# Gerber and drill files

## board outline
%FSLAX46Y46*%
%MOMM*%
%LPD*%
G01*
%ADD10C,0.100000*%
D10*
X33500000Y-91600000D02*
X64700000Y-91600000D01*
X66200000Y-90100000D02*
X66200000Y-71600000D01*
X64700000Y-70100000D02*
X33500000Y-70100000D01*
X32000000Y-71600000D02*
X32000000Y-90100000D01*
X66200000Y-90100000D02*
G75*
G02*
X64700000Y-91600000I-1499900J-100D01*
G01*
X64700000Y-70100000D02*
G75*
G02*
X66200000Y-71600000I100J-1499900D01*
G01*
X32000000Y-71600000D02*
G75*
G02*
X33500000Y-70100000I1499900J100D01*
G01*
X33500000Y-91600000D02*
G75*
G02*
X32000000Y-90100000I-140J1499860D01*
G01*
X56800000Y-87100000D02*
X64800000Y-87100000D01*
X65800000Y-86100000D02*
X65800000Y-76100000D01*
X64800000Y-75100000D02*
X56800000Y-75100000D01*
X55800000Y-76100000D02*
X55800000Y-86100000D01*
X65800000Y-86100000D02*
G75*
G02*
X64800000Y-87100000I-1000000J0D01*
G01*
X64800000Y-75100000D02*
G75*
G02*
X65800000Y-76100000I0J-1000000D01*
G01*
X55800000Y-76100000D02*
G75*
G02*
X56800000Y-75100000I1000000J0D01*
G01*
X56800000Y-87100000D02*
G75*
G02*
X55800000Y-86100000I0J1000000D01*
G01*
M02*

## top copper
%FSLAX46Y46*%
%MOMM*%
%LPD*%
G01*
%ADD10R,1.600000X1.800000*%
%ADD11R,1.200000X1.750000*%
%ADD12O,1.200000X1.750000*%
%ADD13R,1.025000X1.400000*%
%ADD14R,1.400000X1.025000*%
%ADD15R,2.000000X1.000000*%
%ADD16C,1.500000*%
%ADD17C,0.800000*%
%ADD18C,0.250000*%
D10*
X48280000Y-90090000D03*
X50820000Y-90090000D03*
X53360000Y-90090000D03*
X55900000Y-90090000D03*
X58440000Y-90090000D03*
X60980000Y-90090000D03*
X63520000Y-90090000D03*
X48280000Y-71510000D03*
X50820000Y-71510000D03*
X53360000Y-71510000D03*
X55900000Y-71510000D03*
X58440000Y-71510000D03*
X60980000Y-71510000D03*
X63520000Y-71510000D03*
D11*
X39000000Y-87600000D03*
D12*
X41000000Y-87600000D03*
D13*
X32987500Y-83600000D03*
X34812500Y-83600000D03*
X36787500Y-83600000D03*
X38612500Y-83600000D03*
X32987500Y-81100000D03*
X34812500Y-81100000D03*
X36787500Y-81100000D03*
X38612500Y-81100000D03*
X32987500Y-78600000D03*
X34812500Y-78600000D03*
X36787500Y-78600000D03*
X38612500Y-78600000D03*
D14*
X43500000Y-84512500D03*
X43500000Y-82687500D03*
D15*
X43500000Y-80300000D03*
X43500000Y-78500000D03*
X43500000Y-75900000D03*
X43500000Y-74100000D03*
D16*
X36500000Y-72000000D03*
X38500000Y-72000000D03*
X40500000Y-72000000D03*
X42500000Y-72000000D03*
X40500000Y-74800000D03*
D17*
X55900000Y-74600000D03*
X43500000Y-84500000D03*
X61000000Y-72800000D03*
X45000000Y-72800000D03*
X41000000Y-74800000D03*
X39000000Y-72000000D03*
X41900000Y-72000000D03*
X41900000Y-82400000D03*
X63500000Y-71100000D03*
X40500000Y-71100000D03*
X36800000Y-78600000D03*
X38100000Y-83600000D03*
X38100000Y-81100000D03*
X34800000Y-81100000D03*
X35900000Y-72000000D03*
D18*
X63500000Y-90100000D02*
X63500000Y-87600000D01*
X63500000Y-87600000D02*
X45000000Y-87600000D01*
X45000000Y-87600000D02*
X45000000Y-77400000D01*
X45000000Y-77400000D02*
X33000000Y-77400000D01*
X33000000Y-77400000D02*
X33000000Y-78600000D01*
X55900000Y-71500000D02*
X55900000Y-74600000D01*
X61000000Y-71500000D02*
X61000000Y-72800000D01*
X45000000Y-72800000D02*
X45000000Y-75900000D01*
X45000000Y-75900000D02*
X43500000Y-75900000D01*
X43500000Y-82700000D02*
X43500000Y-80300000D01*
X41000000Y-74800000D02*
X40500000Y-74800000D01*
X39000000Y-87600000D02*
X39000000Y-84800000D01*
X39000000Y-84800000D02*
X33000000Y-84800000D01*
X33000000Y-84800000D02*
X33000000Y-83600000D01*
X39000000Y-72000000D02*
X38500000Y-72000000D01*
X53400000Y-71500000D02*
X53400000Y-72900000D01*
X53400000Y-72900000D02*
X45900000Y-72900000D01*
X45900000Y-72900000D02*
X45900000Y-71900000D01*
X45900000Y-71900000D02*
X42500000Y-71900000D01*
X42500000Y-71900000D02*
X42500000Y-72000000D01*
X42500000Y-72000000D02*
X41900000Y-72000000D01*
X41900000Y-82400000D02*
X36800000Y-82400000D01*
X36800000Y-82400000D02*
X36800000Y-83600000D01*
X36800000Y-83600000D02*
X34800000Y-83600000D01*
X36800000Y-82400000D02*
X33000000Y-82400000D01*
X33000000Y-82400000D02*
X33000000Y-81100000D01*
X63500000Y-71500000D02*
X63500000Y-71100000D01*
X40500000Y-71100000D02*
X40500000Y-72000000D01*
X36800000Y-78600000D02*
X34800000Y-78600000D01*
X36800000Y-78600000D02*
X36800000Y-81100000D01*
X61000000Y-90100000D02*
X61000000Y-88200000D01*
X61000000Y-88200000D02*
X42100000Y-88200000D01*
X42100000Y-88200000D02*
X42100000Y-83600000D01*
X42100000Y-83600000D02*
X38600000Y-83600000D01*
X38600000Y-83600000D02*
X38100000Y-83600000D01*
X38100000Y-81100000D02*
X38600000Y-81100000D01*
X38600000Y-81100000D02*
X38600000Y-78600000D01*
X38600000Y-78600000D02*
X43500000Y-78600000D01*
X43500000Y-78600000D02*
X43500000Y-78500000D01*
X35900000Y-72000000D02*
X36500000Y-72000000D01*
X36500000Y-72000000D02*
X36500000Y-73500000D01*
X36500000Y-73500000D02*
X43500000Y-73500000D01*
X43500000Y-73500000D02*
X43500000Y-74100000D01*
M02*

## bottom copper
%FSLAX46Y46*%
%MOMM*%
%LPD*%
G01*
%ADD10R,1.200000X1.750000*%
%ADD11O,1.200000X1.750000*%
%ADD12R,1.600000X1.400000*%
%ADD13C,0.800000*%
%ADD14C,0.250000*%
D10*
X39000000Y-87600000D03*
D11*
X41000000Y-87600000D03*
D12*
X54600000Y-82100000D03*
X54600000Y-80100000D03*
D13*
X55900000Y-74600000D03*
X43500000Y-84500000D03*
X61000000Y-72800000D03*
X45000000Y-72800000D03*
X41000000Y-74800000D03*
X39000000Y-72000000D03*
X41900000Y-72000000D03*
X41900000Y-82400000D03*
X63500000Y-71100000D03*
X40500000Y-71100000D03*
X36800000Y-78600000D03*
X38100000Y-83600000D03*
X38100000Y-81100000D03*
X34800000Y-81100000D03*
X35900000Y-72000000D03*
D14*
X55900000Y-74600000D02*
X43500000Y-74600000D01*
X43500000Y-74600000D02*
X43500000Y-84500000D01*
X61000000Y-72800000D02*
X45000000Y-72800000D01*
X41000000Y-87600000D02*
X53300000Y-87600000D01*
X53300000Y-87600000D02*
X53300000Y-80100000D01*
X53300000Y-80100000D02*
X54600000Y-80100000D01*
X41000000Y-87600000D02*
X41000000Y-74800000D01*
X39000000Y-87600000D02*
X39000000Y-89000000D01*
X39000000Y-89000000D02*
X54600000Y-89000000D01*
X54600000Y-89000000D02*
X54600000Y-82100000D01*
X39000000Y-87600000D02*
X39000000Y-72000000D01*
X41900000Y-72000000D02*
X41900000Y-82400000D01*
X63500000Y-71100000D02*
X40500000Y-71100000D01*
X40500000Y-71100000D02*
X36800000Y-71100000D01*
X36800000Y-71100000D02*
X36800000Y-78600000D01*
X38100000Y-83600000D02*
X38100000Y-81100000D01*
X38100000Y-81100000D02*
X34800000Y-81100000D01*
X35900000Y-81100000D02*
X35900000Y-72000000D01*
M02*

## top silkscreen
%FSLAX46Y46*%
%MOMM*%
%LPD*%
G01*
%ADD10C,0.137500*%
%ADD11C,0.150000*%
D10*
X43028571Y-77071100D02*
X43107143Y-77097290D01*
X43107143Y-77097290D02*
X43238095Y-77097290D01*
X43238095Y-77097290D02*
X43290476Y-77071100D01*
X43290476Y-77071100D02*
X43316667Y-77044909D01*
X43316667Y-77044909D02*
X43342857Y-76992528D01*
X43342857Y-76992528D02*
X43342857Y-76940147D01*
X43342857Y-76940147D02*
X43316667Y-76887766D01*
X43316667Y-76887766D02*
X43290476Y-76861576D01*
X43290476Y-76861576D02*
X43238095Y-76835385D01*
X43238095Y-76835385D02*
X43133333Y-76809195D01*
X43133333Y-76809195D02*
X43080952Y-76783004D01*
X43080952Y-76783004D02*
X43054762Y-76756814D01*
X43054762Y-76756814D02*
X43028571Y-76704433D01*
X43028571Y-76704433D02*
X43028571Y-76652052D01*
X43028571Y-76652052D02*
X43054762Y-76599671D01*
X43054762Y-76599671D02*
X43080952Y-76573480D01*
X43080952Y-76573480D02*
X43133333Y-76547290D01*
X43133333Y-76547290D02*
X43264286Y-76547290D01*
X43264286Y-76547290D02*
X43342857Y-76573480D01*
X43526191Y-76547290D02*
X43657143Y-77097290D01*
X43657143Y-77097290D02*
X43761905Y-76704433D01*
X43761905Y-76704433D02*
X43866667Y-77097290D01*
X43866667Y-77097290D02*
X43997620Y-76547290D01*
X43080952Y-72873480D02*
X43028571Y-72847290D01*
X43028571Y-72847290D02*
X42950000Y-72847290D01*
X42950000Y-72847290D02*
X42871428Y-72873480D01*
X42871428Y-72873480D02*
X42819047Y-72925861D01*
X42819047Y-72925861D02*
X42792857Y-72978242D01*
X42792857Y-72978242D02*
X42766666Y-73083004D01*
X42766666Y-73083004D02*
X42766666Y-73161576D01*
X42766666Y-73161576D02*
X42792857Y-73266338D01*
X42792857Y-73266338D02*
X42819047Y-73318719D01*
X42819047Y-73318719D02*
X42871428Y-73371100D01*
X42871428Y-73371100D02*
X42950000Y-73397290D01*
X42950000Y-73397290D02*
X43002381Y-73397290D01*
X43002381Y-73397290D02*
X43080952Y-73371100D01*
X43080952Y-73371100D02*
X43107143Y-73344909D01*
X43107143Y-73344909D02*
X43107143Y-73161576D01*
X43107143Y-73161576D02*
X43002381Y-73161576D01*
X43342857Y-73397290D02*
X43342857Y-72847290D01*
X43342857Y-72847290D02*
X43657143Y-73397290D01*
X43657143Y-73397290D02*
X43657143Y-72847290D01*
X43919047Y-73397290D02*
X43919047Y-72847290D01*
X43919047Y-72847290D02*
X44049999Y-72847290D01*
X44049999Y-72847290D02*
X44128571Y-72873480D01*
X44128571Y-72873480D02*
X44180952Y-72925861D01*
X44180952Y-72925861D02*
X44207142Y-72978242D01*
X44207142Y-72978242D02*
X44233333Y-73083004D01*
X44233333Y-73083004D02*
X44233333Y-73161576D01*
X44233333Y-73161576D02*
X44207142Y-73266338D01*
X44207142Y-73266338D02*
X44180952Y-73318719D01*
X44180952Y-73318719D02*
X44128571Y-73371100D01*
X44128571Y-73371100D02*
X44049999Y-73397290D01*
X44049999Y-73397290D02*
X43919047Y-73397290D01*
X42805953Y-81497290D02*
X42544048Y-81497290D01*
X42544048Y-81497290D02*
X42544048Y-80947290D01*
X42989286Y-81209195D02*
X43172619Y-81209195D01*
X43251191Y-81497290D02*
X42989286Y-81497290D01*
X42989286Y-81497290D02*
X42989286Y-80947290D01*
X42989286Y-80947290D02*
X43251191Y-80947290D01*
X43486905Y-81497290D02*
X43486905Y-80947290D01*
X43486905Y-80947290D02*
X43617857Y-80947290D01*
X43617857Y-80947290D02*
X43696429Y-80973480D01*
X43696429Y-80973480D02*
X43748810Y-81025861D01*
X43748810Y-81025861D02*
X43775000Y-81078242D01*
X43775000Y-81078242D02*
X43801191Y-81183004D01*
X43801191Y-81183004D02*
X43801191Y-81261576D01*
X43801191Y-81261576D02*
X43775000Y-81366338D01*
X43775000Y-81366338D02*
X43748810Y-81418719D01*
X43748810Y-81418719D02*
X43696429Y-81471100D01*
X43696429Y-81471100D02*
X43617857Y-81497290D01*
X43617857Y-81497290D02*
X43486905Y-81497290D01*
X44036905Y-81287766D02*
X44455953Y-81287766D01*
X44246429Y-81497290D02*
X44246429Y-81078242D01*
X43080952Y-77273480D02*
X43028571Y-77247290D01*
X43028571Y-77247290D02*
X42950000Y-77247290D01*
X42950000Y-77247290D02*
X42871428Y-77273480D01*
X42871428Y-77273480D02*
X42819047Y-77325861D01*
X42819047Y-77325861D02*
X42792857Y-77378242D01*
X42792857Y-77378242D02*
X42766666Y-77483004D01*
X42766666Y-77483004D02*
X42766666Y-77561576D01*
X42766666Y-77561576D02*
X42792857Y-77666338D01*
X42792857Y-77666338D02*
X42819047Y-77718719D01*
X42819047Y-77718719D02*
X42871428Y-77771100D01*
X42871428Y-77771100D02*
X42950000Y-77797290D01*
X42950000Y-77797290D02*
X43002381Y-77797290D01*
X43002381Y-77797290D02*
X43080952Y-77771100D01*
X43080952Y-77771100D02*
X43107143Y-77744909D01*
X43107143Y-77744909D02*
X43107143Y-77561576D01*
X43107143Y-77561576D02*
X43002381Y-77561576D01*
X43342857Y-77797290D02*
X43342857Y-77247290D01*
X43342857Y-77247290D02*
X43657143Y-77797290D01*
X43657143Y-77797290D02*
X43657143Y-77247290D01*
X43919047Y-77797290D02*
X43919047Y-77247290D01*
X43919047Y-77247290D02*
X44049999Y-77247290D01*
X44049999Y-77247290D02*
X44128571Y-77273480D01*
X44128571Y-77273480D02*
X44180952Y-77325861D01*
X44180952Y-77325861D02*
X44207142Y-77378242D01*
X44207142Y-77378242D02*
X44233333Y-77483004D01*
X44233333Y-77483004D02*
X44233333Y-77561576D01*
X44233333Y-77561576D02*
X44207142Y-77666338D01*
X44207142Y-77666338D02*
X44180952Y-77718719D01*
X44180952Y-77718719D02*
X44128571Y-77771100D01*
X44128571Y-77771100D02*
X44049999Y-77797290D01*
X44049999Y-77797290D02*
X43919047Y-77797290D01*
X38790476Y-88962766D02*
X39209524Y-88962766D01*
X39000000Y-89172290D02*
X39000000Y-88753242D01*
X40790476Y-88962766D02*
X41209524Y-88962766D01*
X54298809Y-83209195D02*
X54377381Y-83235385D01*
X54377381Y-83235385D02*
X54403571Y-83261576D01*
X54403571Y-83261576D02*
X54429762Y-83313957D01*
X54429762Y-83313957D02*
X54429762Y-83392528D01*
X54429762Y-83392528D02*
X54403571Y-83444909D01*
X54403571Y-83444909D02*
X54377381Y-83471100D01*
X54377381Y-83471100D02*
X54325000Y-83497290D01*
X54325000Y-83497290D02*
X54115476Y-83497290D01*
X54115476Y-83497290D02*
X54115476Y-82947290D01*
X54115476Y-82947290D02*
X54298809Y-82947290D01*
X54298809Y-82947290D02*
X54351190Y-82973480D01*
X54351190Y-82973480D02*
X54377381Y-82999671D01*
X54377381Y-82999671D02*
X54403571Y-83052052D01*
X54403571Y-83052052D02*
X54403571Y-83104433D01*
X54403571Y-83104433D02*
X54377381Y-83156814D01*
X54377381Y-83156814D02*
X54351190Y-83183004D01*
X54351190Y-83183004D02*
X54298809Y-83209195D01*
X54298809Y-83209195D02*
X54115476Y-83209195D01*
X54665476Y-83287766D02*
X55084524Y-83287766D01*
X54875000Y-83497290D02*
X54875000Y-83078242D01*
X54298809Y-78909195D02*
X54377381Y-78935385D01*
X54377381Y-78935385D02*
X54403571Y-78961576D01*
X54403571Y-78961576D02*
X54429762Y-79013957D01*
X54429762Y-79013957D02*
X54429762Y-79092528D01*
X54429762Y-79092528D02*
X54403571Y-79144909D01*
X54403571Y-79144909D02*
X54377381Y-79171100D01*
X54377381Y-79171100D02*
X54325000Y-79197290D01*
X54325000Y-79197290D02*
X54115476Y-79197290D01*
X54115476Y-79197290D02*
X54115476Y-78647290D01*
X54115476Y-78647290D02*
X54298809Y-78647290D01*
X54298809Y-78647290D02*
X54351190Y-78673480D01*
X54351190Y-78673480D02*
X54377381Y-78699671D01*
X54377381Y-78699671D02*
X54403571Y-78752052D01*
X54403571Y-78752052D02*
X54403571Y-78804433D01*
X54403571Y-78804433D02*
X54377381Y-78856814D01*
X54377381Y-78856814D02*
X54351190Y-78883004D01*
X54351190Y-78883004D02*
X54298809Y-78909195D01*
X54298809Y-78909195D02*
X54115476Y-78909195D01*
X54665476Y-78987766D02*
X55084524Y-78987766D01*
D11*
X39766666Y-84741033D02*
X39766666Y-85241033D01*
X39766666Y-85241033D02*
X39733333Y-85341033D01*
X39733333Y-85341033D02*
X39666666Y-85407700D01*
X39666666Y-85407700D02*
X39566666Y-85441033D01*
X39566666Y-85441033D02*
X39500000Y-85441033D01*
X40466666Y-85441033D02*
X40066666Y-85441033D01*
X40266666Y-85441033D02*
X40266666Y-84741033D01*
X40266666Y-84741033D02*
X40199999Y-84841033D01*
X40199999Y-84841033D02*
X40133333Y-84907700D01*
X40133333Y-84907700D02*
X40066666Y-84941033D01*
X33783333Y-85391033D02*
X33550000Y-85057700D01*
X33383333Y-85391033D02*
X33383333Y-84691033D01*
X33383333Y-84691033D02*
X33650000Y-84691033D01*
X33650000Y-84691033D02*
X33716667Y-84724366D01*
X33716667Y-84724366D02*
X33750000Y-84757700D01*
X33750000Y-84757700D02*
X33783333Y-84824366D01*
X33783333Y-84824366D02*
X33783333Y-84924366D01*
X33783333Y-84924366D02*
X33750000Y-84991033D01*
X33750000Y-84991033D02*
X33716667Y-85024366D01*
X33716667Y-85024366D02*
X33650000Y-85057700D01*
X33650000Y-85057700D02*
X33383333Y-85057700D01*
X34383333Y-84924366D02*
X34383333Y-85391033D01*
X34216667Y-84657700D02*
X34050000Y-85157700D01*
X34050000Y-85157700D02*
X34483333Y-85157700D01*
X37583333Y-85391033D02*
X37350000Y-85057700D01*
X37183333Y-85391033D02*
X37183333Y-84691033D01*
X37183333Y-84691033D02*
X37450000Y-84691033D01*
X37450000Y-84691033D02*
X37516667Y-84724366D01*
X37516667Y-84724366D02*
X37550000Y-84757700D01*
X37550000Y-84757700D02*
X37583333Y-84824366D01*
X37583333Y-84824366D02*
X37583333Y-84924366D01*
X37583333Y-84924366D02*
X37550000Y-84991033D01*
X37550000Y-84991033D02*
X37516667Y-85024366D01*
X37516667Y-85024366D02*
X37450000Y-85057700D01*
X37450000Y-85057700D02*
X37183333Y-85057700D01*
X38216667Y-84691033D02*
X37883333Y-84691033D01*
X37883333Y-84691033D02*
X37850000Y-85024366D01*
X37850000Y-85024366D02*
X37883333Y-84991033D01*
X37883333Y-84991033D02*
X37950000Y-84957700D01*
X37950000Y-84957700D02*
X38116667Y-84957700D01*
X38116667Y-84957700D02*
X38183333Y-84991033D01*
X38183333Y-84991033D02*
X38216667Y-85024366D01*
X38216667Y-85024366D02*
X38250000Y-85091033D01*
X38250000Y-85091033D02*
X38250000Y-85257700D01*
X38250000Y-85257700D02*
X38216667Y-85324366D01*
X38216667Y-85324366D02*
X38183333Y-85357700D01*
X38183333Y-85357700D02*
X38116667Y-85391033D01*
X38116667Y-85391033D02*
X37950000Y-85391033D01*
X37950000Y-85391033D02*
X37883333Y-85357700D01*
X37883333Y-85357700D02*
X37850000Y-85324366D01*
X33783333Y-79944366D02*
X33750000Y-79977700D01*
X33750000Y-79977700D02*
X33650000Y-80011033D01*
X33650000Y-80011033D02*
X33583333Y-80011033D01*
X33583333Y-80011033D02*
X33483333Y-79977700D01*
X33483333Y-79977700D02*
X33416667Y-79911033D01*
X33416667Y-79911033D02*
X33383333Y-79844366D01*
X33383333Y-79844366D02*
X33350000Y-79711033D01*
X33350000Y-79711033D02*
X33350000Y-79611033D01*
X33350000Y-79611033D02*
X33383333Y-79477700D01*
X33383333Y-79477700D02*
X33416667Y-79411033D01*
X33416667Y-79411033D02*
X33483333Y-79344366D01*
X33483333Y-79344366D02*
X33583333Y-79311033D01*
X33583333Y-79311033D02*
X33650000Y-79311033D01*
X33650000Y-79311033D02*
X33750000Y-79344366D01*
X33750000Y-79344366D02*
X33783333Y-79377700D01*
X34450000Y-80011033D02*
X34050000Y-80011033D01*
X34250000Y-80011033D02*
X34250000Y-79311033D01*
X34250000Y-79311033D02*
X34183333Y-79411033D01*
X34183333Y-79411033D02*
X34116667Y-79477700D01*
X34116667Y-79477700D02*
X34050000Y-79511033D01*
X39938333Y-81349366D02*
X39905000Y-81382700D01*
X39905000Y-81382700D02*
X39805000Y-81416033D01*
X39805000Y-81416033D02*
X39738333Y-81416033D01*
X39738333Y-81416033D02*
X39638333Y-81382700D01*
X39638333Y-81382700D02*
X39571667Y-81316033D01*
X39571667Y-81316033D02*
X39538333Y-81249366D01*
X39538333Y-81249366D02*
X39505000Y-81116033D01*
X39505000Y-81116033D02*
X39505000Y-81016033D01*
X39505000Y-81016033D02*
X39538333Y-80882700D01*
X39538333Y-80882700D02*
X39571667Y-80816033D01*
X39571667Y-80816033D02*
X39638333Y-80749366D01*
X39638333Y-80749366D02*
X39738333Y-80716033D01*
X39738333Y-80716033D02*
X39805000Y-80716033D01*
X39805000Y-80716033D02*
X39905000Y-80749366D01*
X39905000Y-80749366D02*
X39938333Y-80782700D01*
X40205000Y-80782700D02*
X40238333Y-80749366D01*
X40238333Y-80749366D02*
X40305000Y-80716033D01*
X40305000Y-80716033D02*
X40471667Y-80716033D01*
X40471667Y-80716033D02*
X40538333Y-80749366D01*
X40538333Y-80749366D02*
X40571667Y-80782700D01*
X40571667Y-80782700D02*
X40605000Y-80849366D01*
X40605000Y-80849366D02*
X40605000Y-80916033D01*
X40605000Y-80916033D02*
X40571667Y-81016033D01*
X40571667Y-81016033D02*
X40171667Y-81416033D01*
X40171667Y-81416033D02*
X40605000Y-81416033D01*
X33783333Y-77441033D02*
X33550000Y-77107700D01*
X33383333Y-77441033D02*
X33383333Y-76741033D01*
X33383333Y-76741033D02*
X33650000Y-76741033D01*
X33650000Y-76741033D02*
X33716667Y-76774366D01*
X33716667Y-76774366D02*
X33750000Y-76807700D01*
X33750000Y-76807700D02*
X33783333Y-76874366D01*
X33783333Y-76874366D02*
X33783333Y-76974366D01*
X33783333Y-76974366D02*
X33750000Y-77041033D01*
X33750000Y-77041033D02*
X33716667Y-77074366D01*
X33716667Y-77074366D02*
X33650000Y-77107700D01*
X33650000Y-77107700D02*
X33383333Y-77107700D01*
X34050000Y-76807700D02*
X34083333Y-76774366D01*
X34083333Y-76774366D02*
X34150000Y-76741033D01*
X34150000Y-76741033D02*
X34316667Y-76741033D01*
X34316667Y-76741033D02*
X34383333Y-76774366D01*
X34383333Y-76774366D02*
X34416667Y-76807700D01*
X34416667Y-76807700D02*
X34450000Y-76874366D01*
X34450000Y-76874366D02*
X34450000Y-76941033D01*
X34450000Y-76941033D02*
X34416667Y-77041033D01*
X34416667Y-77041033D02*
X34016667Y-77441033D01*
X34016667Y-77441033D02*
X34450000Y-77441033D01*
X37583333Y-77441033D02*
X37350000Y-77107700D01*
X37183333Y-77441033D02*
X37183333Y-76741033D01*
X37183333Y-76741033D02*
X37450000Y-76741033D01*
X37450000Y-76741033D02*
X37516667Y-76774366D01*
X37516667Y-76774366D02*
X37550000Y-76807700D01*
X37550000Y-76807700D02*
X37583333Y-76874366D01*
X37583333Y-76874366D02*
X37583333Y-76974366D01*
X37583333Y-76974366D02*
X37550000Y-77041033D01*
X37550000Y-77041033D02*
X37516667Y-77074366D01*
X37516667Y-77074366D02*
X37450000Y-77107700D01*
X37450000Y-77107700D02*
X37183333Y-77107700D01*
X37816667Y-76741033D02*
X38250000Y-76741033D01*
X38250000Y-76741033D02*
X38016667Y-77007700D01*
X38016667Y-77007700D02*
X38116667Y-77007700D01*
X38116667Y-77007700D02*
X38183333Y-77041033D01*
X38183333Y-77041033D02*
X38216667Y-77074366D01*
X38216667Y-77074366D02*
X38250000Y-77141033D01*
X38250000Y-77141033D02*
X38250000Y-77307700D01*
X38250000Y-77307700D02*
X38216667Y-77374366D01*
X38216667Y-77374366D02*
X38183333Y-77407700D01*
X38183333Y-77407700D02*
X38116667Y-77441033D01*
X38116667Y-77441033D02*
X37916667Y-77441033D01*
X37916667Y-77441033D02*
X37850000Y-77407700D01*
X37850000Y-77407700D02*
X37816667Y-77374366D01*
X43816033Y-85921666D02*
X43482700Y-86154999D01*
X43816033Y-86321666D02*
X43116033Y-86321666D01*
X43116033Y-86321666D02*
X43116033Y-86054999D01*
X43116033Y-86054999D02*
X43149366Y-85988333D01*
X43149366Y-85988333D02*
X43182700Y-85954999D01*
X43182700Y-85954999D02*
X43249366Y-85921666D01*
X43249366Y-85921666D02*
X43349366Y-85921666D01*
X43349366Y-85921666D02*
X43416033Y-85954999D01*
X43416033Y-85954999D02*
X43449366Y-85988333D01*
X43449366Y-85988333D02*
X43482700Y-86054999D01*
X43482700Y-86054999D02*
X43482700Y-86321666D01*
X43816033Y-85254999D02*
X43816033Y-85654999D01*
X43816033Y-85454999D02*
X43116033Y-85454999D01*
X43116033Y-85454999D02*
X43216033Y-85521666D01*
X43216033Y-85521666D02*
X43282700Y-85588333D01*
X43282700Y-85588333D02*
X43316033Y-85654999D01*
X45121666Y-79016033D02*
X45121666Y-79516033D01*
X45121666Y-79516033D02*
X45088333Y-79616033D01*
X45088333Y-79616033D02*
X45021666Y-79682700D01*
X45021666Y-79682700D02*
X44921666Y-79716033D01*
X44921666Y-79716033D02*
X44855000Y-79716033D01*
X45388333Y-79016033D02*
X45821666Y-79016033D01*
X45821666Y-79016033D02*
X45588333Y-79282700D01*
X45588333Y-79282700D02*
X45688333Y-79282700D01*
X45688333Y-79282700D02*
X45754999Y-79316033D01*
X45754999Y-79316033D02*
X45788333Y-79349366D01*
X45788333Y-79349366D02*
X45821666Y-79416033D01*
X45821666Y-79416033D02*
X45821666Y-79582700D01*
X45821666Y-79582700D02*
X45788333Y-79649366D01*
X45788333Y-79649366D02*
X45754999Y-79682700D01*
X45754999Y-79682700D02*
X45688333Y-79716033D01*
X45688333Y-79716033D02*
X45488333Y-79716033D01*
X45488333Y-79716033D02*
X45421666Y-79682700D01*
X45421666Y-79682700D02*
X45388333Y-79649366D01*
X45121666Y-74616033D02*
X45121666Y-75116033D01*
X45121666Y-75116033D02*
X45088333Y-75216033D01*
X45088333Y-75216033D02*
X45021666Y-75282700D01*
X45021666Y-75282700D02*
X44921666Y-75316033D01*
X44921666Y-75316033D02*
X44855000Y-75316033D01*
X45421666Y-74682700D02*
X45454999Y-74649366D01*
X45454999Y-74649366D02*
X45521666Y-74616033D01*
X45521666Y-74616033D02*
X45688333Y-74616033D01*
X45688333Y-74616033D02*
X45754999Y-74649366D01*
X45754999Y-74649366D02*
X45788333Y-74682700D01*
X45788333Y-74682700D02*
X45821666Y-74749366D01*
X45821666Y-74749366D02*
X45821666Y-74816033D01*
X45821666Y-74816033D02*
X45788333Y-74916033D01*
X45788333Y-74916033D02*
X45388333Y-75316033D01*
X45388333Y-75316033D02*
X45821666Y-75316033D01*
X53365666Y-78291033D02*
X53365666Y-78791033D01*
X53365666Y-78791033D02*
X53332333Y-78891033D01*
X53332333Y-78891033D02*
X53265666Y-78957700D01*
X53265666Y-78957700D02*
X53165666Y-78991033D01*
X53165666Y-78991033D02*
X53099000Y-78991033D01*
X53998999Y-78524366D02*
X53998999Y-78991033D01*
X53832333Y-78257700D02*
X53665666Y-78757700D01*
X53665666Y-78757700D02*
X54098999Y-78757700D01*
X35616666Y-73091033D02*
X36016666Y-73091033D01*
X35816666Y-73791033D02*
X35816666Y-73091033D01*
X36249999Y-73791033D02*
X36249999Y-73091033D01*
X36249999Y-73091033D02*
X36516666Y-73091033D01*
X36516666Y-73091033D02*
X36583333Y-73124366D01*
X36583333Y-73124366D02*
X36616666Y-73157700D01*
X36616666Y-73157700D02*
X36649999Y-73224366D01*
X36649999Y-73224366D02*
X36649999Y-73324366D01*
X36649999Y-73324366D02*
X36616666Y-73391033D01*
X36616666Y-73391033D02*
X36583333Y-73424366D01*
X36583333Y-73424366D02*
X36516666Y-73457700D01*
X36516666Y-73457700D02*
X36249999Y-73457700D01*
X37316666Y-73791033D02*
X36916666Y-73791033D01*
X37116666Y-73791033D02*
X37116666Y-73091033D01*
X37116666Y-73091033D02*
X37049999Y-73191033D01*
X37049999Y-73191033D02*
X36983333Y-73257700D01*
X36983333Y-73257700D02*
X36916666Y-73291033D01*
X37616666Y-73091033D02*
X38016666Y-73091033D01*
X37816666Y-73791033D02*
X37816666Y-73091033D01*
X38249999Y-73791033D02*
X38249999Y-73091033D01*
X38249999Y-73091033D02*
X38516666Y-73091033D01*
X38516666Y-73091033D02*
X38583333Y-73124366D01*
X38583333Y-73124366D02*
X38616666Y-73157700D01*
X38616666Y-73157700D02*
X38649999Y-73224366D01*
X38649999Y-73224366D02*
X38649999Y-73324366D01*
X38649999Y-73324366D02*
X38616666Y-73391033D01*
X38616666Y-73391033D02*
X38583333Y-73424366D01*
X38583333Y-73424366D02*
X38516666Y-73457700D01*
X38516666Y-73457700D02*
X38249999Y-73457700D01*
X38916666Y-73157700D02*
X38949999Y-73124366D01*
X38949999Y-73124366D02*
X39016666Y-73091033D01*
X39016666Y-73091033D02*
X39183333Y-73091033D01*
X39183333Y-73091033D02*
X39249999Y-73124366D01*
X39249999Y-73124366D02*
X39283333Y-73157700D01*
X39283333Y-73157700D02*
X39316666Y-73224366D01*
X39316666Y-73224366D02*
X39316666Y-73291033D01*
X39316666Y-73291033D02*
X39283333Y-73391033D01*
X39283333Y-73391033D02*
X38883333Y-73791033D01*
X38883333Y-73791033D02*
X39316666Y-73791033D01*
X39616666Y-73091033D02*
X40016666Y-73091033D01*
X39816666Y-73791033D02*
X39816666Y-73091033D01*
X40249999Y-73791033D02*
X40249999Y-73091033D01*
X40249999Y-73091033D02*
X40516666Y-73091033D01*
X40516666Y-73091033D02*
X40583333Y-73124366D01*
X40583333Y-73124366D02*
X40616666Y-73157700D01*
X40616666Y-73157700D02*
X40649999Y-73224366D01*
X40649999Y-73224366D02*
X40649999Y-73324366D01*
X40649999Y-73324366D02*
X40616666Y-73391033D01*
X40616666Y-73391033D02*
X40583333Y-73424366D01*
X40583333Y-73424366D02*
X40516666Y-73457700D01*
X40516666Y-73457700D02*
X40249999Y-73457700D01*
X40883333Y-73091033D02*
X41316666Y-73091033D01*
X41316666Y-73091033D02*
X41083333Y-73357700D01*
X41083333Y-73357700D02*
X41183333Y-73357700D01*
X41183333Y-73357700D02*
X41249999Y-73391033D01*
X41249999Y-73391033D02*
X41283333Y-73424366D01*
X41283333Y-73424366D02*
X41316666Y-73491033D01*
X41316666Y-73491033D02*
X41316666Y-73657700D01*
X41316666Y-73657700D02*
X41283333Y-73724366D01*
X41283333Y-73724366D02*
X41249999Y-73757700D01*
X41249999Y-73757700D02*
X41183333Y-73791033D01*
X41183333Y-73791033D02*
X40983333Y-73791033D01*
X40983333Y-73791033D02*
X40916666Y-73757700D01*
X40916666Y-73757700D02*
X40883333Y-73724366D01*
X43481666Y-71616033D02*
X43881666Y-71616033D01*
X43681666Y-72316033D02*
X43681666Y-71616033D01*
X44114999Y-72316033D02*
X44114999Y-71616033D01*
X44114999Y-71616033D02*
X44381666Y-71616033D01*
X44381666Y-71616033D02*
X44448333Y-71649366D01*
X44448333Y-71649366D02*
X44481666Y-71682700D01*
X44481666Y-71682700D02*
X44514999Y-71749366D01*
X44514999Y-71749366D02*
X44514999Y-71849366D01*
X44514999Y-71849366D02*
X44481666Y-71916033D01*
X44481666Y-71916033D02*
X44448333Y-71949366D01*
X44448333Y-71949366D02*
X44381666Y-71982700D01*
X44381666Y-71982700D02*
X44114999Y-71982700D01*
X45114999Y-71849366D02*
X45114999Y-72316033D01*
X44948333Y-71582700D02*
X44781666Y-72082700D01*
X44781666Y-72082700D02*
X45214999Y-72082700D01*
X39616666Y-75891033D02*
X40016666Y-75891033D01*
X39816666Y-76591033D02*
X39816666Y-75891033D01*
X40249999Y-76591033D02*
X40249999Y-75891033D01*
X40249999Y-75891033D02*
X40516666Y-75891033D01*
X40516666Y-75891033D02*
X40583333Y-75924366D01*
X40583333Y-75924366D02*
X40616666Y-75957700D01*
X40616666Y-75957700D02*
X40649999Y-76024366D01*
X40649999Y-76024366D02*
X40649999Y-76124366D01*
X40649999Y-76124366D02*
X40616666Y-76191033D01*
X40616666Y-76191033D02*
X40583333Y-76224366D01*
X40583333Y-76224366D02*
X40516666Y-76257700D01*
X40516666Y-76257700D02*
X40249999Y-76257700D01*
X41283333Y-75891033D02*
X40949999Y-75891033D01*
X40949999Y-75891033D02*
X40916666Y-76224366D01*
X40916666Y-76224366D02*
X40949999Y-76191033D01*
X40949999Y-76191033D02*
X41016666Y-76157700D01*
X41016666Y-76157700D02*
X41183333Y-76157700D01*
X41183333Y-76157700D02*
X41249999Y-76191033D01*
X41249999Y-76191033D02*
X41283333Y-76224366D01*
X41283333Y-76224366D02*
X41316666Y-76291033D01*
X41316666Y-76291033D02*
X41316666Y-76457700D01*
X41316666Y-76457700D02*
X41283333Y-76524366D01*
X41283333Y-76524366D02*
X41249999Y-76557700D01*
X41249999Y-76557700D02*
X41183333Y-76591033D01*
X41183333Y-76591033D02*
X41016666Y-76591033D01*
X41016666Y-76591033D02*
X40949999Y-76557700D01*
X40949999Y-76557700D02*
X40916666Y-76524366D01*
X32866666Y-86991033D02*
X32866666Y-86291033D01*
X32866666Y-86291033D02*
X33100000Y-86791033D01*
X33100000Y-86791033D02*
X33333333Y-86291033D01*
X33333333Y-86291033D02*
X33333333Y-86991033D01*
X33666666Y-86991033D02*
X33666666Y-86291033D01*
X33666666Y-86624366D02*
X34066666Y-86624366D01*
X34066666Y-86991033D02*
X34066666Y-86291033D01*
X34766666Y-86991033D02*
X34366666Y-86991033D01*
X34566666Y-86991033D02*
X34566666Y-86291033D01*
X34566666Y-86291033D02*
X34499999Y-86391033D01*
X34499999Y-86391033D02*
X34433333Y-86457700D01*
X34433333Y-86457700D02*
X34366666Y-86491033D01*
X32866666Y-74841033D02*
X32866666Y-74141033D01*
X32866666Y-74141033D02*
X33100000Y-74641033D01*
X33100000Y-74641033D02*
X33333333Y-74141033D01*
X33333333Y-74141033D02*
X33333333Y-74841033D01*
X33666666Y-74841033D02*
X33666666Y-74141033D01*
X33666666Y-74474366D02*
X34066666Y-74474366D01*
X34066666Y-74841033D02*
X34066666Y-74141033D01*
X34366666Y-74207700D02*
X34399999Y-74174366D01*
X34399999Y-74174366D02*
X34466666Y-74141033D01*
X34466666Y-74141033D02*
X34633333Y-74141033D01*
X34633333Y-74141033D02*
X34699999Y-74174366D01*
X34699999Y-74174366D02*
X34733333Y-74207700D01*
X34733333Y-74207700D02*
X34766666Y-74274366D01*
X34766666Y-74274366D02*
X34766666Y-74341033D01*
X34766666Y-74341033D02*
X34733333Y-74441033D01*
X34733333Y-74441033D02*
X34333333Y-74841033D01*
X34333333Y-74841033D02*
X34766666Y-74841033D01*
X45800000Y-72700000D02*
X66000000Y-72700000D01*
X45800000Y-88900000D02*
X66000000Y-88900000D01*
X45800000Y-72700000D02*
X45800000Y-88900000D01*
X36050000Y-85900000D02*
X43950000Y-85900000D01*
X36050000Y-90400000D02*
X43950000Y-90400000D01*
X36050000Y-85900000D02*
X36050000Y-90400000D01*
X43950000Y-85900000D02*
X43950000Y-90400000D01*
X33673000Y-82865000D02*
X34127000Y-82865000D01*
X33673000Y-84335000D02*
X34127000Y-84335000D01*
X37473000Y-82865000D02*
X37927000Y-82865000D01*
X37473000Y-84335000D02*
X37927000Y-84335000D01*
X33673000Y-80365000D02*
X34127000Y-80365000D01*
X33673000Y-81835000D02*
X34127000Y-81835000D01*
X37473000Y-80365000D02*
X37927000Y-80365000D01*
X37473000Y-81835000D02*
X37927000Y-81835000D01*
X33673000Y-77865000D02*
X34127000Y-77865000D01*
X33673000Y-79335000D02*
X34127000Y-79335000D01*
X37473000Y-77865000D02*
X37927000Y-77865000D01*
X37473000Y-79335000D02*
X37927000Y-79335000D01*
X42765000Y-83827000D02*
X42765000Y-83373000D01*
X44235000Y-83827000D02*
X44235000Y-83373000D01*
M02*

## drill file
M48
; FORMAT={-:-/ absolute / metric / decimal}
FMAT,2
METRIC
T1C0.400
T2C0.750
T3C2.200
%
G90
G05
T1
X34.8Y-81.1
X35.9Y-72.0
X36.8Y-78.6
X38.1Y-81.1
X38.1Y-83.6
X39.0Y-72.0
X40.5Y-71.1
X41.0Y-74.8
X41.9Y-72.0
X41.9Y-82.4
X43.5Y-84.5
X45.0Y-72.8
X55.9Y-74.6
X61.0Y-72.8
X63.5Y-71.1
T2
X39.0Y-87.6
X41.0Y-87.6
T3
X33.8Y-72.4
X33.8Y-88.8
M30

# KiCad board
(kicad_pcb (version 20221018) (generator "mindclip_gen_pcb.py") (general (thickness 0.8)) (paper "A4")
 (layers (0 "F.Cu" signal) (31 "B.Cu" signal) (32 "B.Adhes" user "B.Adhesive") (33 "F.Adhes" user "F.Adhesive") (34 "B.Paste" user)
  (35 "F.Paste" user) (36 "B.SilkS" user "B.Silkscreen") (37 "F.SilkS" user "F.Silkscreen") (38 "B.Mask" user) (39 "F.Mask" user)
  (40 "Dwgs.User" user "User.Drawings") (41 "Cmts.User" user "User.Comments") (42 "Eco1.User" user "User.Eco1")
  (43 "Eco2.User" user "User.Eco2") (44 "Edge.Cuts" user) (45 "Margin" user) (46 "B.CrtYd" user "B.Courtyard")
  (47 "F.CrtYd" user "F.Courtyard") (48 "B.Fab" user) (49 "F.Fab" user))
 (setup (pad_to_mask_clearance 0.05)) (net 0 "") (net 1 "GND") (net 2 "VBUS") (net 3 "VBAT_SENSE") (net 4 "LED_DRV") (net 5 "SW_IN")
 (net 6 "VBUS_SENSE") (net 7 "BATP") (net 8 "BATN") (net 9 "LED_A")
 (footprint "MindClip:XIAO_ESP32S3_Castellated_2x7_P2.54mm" (layer "F.Cu") (at 55.9 80.8)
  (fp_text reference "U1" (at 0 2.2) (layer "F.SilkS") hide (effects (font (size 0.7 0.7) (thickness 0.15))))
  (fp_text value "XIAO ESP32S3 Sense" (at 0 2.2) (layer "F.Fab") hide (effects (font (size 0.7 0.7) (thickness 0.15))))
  (fp_line (start -10.1 -8.1) (end 10.1 -8.1) (stroke (width 0.15) (type solid)) (layer "F.SilkS"))
  (fp_line (start -10.1 8.1) (end 10.1 8.1) (stroke (width 0.15) (type solid)) (layer "F.SilkS"))
  (fp_line (start -10.1 -8.1) (end -10.1 8.1) (stroke (width 0.15) (type solid)) (layer "F.SilkS"))
  (pad "D7" smd rect (at -7.62 9.29) (size 1.6 1.8) (layers "F.Cu" "F.Paste" "F.Mask"))
  (pad "D8" smd rect (at -5.08 9.29) (size 1.6 1.8) (layers "F.Cu" "F.Paste" "F.Mask"))
  (pad "D9" smd rect (at -2.54 9.29) (size 1.6 1.8) (layers "F.Cu" "F.Paste" "F.Mask"))
  (pad "D10" smd rect (at 0 9.29) (size 1.6 1.8) (layers "F.Cu" "F.Paste" "F.Mask"))
  (pad "3V3" smd rect (at 2.54 9.29) (size 1.6 1.8) (layers "F.Cu" "F.Paste" "F.Mask"))
  (pad "GND" smd rect (at 5.08 9.29) (size 1.6 1.8) (layers "F.Cu" "F.Paste" "F.Mask") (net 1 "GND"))
  (pad "5V" smd rect (at 7.62 9.29) (size 1.6 1.8) (layers "F.Cu" "F.Paste" "F.Mask") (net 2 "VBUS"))
  (pad "D6" smd rect (at -7.62 -9.29) (size 1.6 1.8) (layers "F.Cu" "F.Paste" "F.Mask"))
  (pad "D5" smd rect (at -5.08 -9.29) (size 1.6 1.8) (layers "F.Cu" "F.Paste" "F.Mask"))
  (pad "D4" smd rect (at -2.54 -9.29) (size 1.6 1.8) (layers "F.Cu" "F.Paste" "F.Mask") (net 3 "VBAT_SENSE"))
  (pad "D3" smd rect (at 0 -9.29) (size 1.6 1.8) (layers "F.Cu" "F.Paste" "F.Mask") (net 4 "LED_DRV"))
  (pad "D2" smd rect (at 2.54 -9.29) (size 1.6 1.8) (layers "F.Cu" "F.Paste" "F.Mask"))
  (pad "D1" smd rect (at 5.08 -9.29) (size 1.6 1.8) (layers "F.Cu" "F.Paste" "F.Mask") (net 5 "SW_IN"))
  (pad "D0" smd rect (at 7.62 -9.29) (size 1.6 1.8) (layers "F.Cu" "F.Paste" "F.Mask") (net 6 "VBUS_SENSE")))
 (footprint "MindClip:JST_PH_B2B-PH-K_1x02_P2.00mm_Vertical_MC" (layer "F.Cu") (at 40 87.6)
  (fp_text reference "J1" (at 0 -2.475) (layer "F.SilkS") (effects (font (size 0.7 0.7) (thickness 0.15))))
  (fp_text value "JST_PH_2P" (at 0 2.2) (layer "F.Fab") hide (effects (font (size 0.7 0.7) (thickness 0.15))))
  (fp_line (start -3.95 -1.7) (end 3.95 -1.7) (stroke (width 0.15) (type solid)) (layer "F.SilkS"))
  (fp_line (start -3.95 2.8) (end 3.95 2.8) (stroke (width 0.15) (type solid)) (layer "F.SilkS"))
  (fp_line (start -3.95 -1.7) (end -3.95 2.8) (stroke (width 0.15) (type solid)) (layer "F.SilkS"))
  (fp_line (start 3.95 -1.7) (end 3.95 2.8) (stroke (width 0.15) (type solid)) (layer "F.SilkS"))
  (pad "1" thru_hole rect (at -1 0) (size 1.2 1.75) (drill 0.75) (layers "*.Cu" "*.Mask") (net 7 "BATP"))
  (pad "2" thru_hole oval (at 1 0) (size 1.2 1.75) (drill 0.75) (layers "*.Cu" "*.Mask") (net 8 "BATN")))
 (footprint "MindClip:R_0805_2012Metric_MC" (layer "F.Cu") (at 33.9 83.6)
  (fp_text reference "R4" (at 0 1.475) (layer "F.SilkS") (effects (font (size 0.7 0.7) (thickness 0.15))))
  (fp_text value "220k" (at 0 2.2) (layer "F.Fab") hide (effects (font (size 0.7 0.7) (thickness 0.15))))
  (fp_line (start -0.227 -0.735) (end 0.227 -0.735) (stroke (width 0.15) (type solid)) (layer "F.SilkS"))
  (fp_line (start -0.227 0.735) (end 0.227 0.735) (stroke (width 0.15) (type solid)) (layer "F.SilkS"))
  (pad "1" smd rect (at -0.9125 0) (size 1.025 1.4) (layers "F.Cu" "F.Paste" "F.Mask") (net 7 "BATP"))
  (pad "2" smd rect (at 0.9125 0) (size 1.025 1.4) (layers "F.Cu" "F.Paste" "F.Mask") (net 3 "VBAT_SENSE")))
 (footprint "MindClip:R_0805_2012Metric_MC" (layer "F.Cu") (at 37.7 83.6)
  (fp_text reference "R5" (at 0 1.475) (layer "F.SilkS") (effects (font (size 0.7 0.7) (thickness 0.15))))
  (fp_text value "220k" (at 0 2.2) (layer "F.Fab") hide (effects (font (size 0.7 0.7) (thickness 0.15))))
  (fp_line (start -0.227 -0.735) (end 0.227 -0.735) (stroke (width 0.15) (type solid)) (layer "F.SilkS"))
  (fp_line (start -0.227 0.735) (end 0.227 0.735) (stroke (width 0.15) (type solid)) (layer "F.SilkS"))
  (pad "1" smd rect (at -0.9125 0) (size 1.025 1.4) (layers "F.Cu" "F.Paste" "F.Mask") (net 3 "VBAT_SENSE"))
  (pad "2" smd rect (at 0.9125 0) (size 1.025 1.4) (layers "F.Cu" "F.Paste" "F.Mask") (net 1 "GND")))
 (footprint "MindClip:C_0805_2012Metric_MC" (layer "F.Cu") (at 33.9 81.1)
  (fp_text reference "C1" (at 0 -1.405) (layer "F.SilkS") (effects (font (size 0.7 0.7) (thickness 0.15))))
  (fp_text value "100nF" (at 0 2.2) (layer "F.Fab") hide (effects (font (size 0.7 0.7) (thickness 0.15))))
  (fp_line (start -0.227 -0.735) (end 0.227 -0.735) (stroke (width 0.15) (type solid)) (layer "F.SilkS"))
  (fp_line (start -0.227 0.735) (end 0.227 0.735) (stroke (width 0.15) (type solid)) (layer "F.SilkS"))
  (pad "1" smd rect (at -0.9125 0) (size 1.025 1.4) (layers "F.Cu" "F.Paste" "F.Mask") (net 3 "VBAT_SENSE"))
  (pad "2" smd rect (at 0.9125 0) (size 1.025 1.4) (layers "F.Cu" "F.Paste" "F.Mask") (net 1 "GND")))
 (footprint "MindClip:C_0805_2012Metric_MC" (layer "F.Cu") (at 37.7 81.1)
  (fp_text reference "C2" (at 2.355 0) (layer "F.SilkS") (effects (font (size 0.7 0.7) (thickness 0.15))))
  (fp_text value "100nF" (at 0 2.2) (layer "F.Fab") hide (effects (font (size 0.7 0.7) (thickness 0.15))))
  (fp_line (start -0.227 -0.735) (end 0.227 -0.735) (stroke (width 0.15) (type solid)) (layer "F.SilkS"))
  (fp_line (start -0.227 0.735) (end 0.227 0.735) (stroke (width 0.15) (type solid)) (layer "F.SilkS"))
  (pad "1" smd rect (at -0.9125 0) (size 1.025 1.4) (layers "F.Cu" "F.Paste" "F.Mask") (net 6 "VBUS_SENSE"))
  (pad "2" smd rect (at 0.9125 0) (size 1.025 1.4) (layers "F.Cu" "F.Paste" "F.Mask") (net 1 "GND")))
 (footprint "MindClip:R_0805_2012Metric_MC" (layer "F.Cu") (at 33.9 78.6)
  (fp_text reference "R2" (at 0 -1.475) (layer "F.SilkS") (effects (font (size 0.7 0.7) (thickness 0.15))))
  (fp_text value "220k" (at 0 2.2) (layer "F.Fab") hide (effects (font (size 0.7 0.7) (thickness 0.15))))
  (fp_line (start -0.227 -0.735) (end 0.227 -0.735) (stroke (width 0.15) (type solid)) (layer "F.SilkS"))
  (fp_line (start -0.227 0.735) (end 0.227 0.735) (stroke (width 0.15) (type solid)) (layer "F.SilkS"))
  (pad "1" smd rect (at -0.9125 0) (size 1.025 1.4) (layers "F.Cu" "F.Paste" "F.Mask") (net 2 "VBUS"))
  (pad "2" smd rect (at 0.9125 0) (size 1.025 1.4) (layers "F.Cu" "F.Paste" "F.Mask") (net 6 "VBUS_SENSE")))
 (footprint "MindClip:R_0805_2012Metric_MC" (layer "F.Cu") (at 37.7 78.6)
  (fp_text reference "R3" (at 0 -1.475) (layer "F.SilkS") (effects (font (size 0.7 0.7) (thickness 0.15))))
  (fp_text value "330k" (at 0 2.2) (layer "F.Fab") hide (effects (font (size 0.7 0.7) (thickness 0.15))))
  (fp_line (start -0.227 -0.735) (end 0.227 -0.735) (stroke (width 0.15) (type solid)) (layer "F.SilkS"))
  (fp_line (start -0.227 0.735) (end 0.227 0.735) (stroke (width 0.15) (type solid)) (layer "F.SilkS"))
  (pad "1" smd rect (at -0.9125 0) (size 1.025 1.4) (layers "F.Cu" "F.Paste" "F.Mask") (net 6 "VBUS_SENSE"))
  (pad "2" smd rect (at 0.9125 0) (size 1.025 1.4) (layers "F.Cu" "F.Paste" "F.Mask") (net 1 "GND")))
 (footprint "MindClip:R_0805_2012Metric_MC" (layer "F.Cu") (at 43.5 83.6 90)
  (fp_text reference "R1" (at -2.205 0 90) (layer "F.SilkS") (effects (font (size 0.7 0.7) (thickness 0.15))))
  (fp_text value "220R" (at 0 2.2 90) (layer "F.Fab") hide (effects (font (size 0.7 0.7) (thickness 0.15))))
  (fp_line (start -0.227 -0.735) (end 0.227 -0.735) (stroke (width 0.15) (type solid)) (layer "F.SilkS"))
  (fp_line (start -0.227 0.735) (end 0.227 0.735) (stroke (width 0.15) (type solid)) (layer "F.SilkS"))
  (pad "1" smd rect (at -0.9125 0 90) (size 1.025 1.4) (layers "F.Cu" "F.Paste" "F.Mask") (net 4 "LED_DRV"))
  (pad "2" smd rect (at 0.9125 0 90) (size 1.025 1.4) (layers "F.Cu" "F.Paste" "F.Mask") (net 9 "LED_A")))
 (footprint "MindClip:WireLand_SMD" (layer "F.Cu") (at 43.5 79.4)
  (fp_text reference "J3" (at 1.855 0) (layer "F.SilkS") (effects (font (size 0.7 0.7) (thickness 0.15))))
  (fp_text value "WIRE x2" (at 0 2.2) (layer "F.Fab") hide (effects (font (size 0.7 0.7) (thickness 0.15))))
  (pad "1" smd rect (at 0 0.9) (size 2 1) (layers "F.Cu" "F.Paste" "F.Mask") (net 9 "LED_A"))
  (pad "2" smd rect (at 0 -0.9) (size 2 1) (layers "F.Cu" "F.Paste" "F.Mask") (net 1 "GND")))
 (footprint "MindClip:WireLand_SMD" (layer "F.Cu") (at 43.5 75)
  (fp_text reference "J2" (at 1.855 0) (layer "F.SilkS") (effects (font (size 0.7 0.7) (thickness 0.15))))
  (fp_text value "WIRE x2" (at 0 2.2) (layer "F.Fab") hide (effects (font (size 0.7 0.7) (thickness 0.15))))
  (pad "1" smd rect (at 0 0.9) (size 2 1) (layers "F.Cu" "F.Paste" "F.Mask") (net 5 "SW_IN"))
  (pad "2" smd rect (at 0 -0.9) (size 2 1) (layers "F.Cu" "F.Paste" "F.Mask") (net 1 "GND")))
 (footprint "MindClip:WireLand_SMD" (layer "F.Cu") (at 54.6 81.1)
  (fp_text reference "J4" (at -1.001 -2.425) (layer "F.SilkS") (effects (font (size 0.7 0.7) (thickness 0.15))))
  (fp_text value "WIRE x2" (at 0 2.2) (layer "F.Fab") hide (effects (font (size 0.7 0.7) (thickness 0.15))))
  (pad "1" smd rect (at 0 1) (size 1.6 1.4) (layers "B.Cu" "B.Paste" "B.Mask") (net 7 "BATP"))
  (pad "2" smd rect (at 0 -1) (size 1.6 1.4) (layers "B.Cu" "B.Paste" "B.Mask") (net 8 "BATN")))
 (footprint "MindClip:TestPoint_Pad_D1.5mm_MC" (layer "F.Cu") (at 36.5 72)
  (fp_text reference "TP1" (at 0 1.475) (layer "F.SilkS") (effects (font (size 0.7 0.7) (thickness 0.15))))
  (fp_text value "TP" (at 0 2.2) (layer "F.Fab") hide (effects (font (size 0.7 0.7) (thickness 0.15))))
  (pad "1" smd circle (at 0 0) (size 1.5 1.5) (layers "F.Cu" "F.Paste" "F.Mask") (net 1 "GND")))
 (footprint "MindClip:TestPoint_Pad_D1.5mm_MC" (layer "F.Cu") (at 38.5 72)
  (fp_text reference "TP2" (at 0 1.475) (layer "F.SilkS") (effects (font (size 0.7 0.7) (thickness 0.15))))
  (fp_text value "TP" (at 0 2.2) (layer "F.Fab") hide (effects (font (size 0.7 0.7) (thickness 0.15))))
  (pad "1" smd circle (at 0 0) (size 1.5 1.5) (layers "F.Cu" "F.Paste" "F.Mask") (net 7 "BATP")))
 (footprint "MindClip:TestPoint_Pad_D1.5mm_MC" (layer "F.Cu") (at 40.5 72)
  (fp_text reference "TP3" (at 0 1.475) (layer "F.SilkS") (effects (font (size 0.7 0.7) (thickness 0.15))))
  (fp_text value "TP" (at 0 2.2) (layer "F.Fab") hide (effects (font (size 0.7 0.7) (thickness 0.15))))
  (pad "1" smd circle (at 0 0) (size 1.5 1.5) (layers "F.Cu" "F.Paste" "F.Mask") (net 6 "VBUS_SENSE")))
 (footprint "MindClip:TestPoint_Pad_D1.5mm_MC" (layer "F.Cu") (at 42.5 72)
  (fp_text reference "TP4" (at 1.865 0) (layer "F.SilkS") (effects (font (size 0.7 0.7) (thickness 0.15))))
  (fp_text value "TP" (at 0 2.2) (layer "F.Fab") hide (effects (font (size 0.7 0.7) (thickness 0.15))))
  (pad "1" smd circle (at 0 0) (size 1.5 1.5) (layers "F.Cu" "F.Paste" "F.Mask") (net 3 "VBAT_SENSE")))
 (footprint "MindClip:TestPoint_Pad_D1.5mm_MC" (layer "F.Cu") (at 40.5 74.8)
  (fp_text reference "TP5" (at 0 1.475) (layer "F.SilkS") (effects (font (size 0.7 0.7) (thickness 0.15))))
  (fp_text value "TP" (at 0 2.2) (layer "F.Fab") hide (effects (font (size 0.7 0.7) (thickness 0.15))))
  (pad "1" smd circle (at 0 0) (size 1.5 1.5) (layers "F.Cu" "F.Paste" "F.Mask") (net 8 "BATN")))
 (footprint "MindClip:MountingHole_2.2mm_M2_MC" (layer "F.Cu") (at 33.8 88.8)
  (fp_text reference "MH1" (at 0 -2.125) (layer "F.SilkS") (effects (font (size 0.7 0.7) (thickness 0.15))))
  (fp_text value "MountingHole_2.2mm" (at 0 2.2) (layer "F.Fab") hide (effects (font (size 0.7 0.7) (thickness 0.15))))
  (pad "" np_thru_hole circle (at 0 0) (size 2.2 2.2) (drill 2.2) (layers "F&B.Cu" "*.Mask")))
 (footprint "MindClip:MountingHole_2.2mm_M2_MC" (layer "F.Cu") (at 33.8 72.4)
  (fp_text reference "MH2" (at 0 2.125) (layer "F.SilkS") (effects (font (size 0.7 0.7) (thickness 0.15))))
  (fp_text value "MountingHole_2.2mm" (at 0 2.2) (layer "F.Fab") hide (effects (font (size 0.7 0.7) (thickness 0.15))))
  (pad "" np_thru_hole circle (at 0 0) (size 2.2 2.2) (drill 2.2) (layers "F&B.Cu" "*.Mask")))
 (gr_line (start 33.5 91.6) (end 64.7 91.6) (stroke (width 0.1) (type solid)) (layer "Edge.Cuts"))
 (gr_line (start 66.2 90.1) (end 66.2 71.6) (stroke (width 0.1) (type solid)) (layer "Edge.Cuts"))
 (gr_line (start 64.7 70.1) (end 33.5 70.1) (stroke (width 0.1) (type solid)) (layer "Edge.Cuts"))
 (gr_line (start 32 71.6) (end 32 90.1) (stroke (width 0.1) (type solid)) (layer "Edge.Cuts"))
 (gr_arc (start 64.7 91.6) (mid 65.7607 91.1607) (end 66.2 90.1) (stroke (width 0.1) (type solid)) (layer "Edge.Cuts"))
 (gr_arc (start 66.2 71.6) (mid 65.7607 70.5393) (end 64.7 70.1) (stroke (width 0.1) (type solid)) (layer "Edge.Cuts"))
 (gr_arc (start 33.5 70.1) (mid 32.4393 70.5393) (end 32 71.6) (stroke (width 0.1) (type solid)) (layer "Edge.Cuts"))
 (gr_arc (start 32 90.1) (mid 32.4393 91.1607) (end 33.5 91.6) (stroke (width 0.1) (type solid)) (layer "Edge.Cuts"))
 (gr_line (start 56.8 87.1) (end 64.8 87.1) (stroke (width 0.1) (type solid)) (layer "Edge.Cuts"))
 (gr_line (start 65.8 86.1) (end 65.8 76.1) (stroke (width 0.1) (type solid)) (layer "Edge.Cuts"))
 (gr_line (start 64.8 75.1) (end 56.8 75.1) (stroke (width 0.1) (type solid)) (layer "Edge.Cuts"))
 (gr_line (start 55.8 76.1) (end 55.8 86.1) (stroke (width 0.1) (type solid)) (layer "Edge.Cuts"))
 (gr_arc (start 64.8 87.1) (mid 65.5071 86.8071) (end 65.8 86.1) (stroke (width 0.1) (type solid)) (layer "Edge.Cuts"))
 (gr_arc (start 65.8 76.1) (mid 65.5071 75.3929) (end 64.8 75.1) (stroke (width 0.1) (type solid)) (layer "Edge.Cuts"))
 (gr_arc (start 56.8 75.1) (mid 56.0929 75.3929) (end 55.8 76.1) (stroke (width 0.1) (type solid)) (layer "Edge.Cuts"))
 (gr_arc (start 55.8 86.1) (mid 56.0929 86.8071) (end 56.8 87.1) (stroke (width 0.1) (type solid)) (layer "Edge.Cuts"))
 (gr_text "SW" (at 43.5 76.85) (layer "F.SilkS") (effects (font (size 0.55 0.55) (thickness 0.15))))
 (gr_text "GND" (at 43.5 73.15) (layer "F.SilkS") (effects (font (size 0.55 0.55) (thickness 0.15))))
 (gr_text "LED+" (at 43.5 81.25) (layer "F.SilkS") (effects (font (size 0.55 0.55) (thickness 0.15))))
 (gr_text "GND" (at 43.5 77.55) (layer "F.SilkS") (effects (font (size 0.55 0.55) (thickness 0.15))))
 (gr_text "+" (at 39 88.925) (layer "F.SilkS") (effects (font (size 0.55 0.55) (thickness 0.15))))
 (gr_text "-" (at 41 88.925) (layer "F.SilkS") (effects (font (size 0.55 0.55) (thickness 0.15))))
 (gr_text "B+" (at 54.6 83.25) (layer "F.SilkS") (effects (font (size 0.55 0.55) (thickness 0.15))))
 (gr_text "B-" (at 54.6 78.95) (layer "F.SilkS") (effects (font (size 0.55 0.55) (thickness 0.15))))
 (segment (start 63.5 90.1) (end 63.5 87.6) (width 0.25) (layer "F.Cu") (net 2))
 (segment (start 63.5 87.6) (end 45 87.6) (width 0.25) (layer "F.Cu") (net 2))
 (segment (start 45 87.6) (end 45 77.4) (width 0.25) (layer "F.Cu") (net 2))
 (segment (start 45 77.4) (end 33 77.4) (width 0.25) (layer "F.Cu") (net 2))
 (segment (start 33 77.4) (end 33 78.6) (width 0.25) (layer "F.Cu") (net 2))
 (segment (start 55.9 71.5) (end 55.9 74.6) (width 0.25) (layer "F.Cu") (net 4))
 (segment (start 55.9 74.6) (end 43.5 74.6) (width 0.25) (layer "B.Cu") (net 4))
 (segment (start 43.5 74.6) (end 43.5 84.5) (width 0.25) (layer "B.Cu") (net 4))
 (segment (start 61 71.5) (end 61 72.8) (width 0.25) (layer "F.Cu") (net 5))
 (segment (start 61 72.8) (end 45 72.8) (width 0.25) (layer "B.Cu") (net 5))
 (segment (start 45 72.8) (end 45 75.9) (width 0.25) (layer "F.Cu") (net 5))
 (segment (start 45 75.9) (end 43.5 75.9) (width 0.25) (layer "F.Cu") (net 5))
 (segment (start 43.5 82.7) (end 43.5 80.3) (width 0.25) (layer "F.Cu") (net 9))
 (segment (start 41 87.6) (end 53.3 87.6) (width 0.25) (layer "B.Cu") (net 8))
 (segment (start 53.3 87.6) (end 53.3 80.1) (width 0.25) (layer "B.Cu") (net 8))
 (segment (start 53.3 80.1) (end 54.6 80.1) (width 0.25) (layer "B.Cu") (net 8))
 (segment (start 41 87.6) (end 41 74.8) (width 0.25) (layer "B.Cu") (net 8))
 (segment (start 41 74.8) (end 40.5 74.8) (width 0.25) (layer "F.Cu") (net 8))
 (segment (start 39 87.6) (end 39 84.8) (width 0.25) (layer "F.Cu") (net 7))
 (segment (start 39 84.8) (end 33 84.8) (width 0.25) (layer "F.Cu") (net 7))
 (segment (start 33 84.8) (end 33 83.6) (width 0.25) (layer "F.Cu") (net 7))
 (segment (start 39 87.6) (end 39 89) (width 0.25) (layer "B.Cu") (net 7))
 (segment (start 39 89) (end 54.6 89) (width 0.25) (layer "B.Cu") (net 7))
 (segment (start 54.6 89) (end 54.6 82.1) (width 0.25) (layer "B.Cu") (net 7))
 (segment (start 39 87.6) (end 39 72) (width 0.25) (layer "B.Cu") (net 7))
 (segment (start 39 72) (end 38.5 72) (width 0.25) (layer "F.Cu") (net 7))
 (segment (start 53.4 71.5) (end 53.4 72.9) (width 0.25) (layer "F.Cu") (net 3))
 (segment (start 53.4 72.9) (end 45.9 72.9) (width 0.25) (layer "F.Cu") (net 3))
 (segment (start 45.9 72.9) (end 45.9 71.9) (width 0.25) (layer "F.Cu") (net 3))
 (segment (start 45.9 71.9) (end 42.5 71.9) (width 0.25) (layer "F.Cu") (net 3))
 (segment (start 42.5 71.9) (end 42.5 72) (width 0.25) (layer "F.Cu") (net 3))
 (segment (start 42.5 72) (end 41.9 72) (width 0.25) (layer "F.Cu") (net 3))
 (segment (start 41.9 72) (end 41.9 82.4) (width 0.25) (layer "B.Cu") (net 3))
 (segment (start 41.9 82.4) (end 36.8 82.4) (width 0.25) (layer "F.Cu") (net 3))
 (segment (start 36.8 82.4) (end 36.8 83.6) (width 0.25) (layer "F.Cu") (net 3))
 (segment (start 36.8 83.6) (end 34.8 83.6) (width 0.25) (layer "F.Cu") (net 3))
 (segment (start 36.8 82.4) (end 33 82.4) (width 0.25) (layer "F.Cu") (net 3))
 (segment (start 33 82.4) (end 33 81.1) (width 0.25) (layer "F.Cu") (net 3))
 (segment (start 63.5 71.5) (end 63.5 71.1) (width 0.25) (layer "F.Cu") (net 6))
 (segment (start 63.5 71.1) (end 40.5 71.1) (width 0.25) (layer "B.Cu") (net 6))
 (segment (start 40.5 71.1) (end 40.5 72) (width 0.25) (layer "F.Cu") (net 6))
 (segment (start 40.5 71.1) (end 36.8 71.1) (width 0.25) (layer "B.Cu") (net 6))
 (segment (start 36.8 71.1) (end 36.8 78.6) (width 0.25) (layer "B.Cu") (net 6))
 (segment (start 36.8 78.6) (end 34.8 78.6) (width 0.25) (layer "F.Cu") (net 6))
 (segment (start 36.8 78.6) (end 36.8 81.1) (width 0.25) (layer "F.Cu") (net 6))
 (segment (start 61 90.1) (end 61 88.2) (width 0.25) (layer "F.Cu") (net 1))
 (segment (start 61 88.2) (end 42.1 88.2) (width 0.25) (layer "F.Cu") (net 1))
 (segment (start 42.1 88.2) (end 42.1 83.6) (width 0.25) (layer "F.Cu") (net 1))
 (segment (start 42.1 83.6) (end 38.6 83.6) (width 0.25) (layer "F.Cu") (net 1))
 (segment (start 38.6 83.6) (end 38.1 83.6) (width 0.25) (layer "F.Cu") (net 1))
 (segment (start 38.1 83.6) (end 38.1 81.1) (width 0.25) (layer "B.Cu") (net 1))
 (segment (start 38.1 81.1) (end 38.6 81.1) (width 0.25) (layer "F.Cu") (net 1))
 (segment (start 38.6 81.1) (end 38.6 78.6) (width 0.25) (layer "F.Cu") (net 1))
 (segment (start 38.6 78.6) (end 43.5 78.6) (width 0.25) (layer "F.Cu") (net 1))
 (segment (start 43.5 78.6) (end 43.5 78.5) (width 0.25) (layer "F.Cu") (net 1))
 (segment (start 38.1 81.1) (end 34.8 81.1) (width 0.25) (layer "B.Cu") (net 1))
 (segment (start 35.9 81.1) (end 35.9 72) (width 0.25) (layer "B.Cu") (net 1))
 (segment (start 35.9 72) (end 36.5 72) (width 0.25) (layer "F.Cu") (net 1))
 (segment (start 36.5 72) (end 36.5 73.5) (width 0.25) (layer "F.Cu") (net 1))
 (segment (start 36.5 73.5) (end 43.5 73.5) (width 0.25) (layer "F.Cu") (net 1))
 (segment (start 43.5 73.5) (end 43.5 74.1) (width 0.25) (layer "F.Cu") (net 1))
 (via (at 55.9 74.6) (size 0.8) (drill 0.4) (layers "F.Cu" "B.Cu") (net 4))
 (via (at 43.5 84.5) (size 0.8) (drill 0.4) (layers "F.Cu" "B.Cu") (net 4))
 (via (at 61 72.8) (size 0.8) (drill 0.4) (layers "F.Cu" "B.Cu") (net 5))
 (via (at 45 72.8) (size 0.8) (drill 0.4) (layers "F.Cu" "B.Cu") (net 5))
 (via (at 41 74.8) (size 0.8) (drill 0.4) (layers "F.Cu" "B.Cu") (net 8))
 (via (at 39 72) (size 0.8) (drill 0.4) (layers "F.Cu" "B.Cu") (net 7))
 (via (at 41.9 72) (size 0.8) (drill 0.4) (layers "F.Cu" "B.Cu") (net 3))
 (via (at 41.9 82.4) (size 0.8) (drill 0.4) (layers "F.Cu" "B.Cu") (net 3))
 (via (at 63.5 71.1) (size 0.8) (drill 0.4) (layers "F.Cu" "B.Cu") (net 6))
 (via (at 40.5 71.1) (size 0.8) (drill 0.4) (layers "F.Cu" "B.Cu") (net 6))
 (via (at 36.8 78.6) (size 0.8) (drill 0.4) (layers "F.Cu" "B.Cu") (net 6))
 (via (at 38.1 83.6) (size 0.8) (drill 0.4) (layers "F.Cu" "B.Cu") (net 1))
 (via (at 38.1 81.1) (size 0.8) (drill 0.4) (layers "F.Cu" "B.Cu") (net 1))
 (via (at 34.8 81.1) (size 0.8) (drill 0.4) (layers "F.Cu" "B.Cu") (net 1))
 (via (at 35.9 72) (size 0.8) (drill 0.4) (layers "F.Cu" "B.Cu") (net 1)))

